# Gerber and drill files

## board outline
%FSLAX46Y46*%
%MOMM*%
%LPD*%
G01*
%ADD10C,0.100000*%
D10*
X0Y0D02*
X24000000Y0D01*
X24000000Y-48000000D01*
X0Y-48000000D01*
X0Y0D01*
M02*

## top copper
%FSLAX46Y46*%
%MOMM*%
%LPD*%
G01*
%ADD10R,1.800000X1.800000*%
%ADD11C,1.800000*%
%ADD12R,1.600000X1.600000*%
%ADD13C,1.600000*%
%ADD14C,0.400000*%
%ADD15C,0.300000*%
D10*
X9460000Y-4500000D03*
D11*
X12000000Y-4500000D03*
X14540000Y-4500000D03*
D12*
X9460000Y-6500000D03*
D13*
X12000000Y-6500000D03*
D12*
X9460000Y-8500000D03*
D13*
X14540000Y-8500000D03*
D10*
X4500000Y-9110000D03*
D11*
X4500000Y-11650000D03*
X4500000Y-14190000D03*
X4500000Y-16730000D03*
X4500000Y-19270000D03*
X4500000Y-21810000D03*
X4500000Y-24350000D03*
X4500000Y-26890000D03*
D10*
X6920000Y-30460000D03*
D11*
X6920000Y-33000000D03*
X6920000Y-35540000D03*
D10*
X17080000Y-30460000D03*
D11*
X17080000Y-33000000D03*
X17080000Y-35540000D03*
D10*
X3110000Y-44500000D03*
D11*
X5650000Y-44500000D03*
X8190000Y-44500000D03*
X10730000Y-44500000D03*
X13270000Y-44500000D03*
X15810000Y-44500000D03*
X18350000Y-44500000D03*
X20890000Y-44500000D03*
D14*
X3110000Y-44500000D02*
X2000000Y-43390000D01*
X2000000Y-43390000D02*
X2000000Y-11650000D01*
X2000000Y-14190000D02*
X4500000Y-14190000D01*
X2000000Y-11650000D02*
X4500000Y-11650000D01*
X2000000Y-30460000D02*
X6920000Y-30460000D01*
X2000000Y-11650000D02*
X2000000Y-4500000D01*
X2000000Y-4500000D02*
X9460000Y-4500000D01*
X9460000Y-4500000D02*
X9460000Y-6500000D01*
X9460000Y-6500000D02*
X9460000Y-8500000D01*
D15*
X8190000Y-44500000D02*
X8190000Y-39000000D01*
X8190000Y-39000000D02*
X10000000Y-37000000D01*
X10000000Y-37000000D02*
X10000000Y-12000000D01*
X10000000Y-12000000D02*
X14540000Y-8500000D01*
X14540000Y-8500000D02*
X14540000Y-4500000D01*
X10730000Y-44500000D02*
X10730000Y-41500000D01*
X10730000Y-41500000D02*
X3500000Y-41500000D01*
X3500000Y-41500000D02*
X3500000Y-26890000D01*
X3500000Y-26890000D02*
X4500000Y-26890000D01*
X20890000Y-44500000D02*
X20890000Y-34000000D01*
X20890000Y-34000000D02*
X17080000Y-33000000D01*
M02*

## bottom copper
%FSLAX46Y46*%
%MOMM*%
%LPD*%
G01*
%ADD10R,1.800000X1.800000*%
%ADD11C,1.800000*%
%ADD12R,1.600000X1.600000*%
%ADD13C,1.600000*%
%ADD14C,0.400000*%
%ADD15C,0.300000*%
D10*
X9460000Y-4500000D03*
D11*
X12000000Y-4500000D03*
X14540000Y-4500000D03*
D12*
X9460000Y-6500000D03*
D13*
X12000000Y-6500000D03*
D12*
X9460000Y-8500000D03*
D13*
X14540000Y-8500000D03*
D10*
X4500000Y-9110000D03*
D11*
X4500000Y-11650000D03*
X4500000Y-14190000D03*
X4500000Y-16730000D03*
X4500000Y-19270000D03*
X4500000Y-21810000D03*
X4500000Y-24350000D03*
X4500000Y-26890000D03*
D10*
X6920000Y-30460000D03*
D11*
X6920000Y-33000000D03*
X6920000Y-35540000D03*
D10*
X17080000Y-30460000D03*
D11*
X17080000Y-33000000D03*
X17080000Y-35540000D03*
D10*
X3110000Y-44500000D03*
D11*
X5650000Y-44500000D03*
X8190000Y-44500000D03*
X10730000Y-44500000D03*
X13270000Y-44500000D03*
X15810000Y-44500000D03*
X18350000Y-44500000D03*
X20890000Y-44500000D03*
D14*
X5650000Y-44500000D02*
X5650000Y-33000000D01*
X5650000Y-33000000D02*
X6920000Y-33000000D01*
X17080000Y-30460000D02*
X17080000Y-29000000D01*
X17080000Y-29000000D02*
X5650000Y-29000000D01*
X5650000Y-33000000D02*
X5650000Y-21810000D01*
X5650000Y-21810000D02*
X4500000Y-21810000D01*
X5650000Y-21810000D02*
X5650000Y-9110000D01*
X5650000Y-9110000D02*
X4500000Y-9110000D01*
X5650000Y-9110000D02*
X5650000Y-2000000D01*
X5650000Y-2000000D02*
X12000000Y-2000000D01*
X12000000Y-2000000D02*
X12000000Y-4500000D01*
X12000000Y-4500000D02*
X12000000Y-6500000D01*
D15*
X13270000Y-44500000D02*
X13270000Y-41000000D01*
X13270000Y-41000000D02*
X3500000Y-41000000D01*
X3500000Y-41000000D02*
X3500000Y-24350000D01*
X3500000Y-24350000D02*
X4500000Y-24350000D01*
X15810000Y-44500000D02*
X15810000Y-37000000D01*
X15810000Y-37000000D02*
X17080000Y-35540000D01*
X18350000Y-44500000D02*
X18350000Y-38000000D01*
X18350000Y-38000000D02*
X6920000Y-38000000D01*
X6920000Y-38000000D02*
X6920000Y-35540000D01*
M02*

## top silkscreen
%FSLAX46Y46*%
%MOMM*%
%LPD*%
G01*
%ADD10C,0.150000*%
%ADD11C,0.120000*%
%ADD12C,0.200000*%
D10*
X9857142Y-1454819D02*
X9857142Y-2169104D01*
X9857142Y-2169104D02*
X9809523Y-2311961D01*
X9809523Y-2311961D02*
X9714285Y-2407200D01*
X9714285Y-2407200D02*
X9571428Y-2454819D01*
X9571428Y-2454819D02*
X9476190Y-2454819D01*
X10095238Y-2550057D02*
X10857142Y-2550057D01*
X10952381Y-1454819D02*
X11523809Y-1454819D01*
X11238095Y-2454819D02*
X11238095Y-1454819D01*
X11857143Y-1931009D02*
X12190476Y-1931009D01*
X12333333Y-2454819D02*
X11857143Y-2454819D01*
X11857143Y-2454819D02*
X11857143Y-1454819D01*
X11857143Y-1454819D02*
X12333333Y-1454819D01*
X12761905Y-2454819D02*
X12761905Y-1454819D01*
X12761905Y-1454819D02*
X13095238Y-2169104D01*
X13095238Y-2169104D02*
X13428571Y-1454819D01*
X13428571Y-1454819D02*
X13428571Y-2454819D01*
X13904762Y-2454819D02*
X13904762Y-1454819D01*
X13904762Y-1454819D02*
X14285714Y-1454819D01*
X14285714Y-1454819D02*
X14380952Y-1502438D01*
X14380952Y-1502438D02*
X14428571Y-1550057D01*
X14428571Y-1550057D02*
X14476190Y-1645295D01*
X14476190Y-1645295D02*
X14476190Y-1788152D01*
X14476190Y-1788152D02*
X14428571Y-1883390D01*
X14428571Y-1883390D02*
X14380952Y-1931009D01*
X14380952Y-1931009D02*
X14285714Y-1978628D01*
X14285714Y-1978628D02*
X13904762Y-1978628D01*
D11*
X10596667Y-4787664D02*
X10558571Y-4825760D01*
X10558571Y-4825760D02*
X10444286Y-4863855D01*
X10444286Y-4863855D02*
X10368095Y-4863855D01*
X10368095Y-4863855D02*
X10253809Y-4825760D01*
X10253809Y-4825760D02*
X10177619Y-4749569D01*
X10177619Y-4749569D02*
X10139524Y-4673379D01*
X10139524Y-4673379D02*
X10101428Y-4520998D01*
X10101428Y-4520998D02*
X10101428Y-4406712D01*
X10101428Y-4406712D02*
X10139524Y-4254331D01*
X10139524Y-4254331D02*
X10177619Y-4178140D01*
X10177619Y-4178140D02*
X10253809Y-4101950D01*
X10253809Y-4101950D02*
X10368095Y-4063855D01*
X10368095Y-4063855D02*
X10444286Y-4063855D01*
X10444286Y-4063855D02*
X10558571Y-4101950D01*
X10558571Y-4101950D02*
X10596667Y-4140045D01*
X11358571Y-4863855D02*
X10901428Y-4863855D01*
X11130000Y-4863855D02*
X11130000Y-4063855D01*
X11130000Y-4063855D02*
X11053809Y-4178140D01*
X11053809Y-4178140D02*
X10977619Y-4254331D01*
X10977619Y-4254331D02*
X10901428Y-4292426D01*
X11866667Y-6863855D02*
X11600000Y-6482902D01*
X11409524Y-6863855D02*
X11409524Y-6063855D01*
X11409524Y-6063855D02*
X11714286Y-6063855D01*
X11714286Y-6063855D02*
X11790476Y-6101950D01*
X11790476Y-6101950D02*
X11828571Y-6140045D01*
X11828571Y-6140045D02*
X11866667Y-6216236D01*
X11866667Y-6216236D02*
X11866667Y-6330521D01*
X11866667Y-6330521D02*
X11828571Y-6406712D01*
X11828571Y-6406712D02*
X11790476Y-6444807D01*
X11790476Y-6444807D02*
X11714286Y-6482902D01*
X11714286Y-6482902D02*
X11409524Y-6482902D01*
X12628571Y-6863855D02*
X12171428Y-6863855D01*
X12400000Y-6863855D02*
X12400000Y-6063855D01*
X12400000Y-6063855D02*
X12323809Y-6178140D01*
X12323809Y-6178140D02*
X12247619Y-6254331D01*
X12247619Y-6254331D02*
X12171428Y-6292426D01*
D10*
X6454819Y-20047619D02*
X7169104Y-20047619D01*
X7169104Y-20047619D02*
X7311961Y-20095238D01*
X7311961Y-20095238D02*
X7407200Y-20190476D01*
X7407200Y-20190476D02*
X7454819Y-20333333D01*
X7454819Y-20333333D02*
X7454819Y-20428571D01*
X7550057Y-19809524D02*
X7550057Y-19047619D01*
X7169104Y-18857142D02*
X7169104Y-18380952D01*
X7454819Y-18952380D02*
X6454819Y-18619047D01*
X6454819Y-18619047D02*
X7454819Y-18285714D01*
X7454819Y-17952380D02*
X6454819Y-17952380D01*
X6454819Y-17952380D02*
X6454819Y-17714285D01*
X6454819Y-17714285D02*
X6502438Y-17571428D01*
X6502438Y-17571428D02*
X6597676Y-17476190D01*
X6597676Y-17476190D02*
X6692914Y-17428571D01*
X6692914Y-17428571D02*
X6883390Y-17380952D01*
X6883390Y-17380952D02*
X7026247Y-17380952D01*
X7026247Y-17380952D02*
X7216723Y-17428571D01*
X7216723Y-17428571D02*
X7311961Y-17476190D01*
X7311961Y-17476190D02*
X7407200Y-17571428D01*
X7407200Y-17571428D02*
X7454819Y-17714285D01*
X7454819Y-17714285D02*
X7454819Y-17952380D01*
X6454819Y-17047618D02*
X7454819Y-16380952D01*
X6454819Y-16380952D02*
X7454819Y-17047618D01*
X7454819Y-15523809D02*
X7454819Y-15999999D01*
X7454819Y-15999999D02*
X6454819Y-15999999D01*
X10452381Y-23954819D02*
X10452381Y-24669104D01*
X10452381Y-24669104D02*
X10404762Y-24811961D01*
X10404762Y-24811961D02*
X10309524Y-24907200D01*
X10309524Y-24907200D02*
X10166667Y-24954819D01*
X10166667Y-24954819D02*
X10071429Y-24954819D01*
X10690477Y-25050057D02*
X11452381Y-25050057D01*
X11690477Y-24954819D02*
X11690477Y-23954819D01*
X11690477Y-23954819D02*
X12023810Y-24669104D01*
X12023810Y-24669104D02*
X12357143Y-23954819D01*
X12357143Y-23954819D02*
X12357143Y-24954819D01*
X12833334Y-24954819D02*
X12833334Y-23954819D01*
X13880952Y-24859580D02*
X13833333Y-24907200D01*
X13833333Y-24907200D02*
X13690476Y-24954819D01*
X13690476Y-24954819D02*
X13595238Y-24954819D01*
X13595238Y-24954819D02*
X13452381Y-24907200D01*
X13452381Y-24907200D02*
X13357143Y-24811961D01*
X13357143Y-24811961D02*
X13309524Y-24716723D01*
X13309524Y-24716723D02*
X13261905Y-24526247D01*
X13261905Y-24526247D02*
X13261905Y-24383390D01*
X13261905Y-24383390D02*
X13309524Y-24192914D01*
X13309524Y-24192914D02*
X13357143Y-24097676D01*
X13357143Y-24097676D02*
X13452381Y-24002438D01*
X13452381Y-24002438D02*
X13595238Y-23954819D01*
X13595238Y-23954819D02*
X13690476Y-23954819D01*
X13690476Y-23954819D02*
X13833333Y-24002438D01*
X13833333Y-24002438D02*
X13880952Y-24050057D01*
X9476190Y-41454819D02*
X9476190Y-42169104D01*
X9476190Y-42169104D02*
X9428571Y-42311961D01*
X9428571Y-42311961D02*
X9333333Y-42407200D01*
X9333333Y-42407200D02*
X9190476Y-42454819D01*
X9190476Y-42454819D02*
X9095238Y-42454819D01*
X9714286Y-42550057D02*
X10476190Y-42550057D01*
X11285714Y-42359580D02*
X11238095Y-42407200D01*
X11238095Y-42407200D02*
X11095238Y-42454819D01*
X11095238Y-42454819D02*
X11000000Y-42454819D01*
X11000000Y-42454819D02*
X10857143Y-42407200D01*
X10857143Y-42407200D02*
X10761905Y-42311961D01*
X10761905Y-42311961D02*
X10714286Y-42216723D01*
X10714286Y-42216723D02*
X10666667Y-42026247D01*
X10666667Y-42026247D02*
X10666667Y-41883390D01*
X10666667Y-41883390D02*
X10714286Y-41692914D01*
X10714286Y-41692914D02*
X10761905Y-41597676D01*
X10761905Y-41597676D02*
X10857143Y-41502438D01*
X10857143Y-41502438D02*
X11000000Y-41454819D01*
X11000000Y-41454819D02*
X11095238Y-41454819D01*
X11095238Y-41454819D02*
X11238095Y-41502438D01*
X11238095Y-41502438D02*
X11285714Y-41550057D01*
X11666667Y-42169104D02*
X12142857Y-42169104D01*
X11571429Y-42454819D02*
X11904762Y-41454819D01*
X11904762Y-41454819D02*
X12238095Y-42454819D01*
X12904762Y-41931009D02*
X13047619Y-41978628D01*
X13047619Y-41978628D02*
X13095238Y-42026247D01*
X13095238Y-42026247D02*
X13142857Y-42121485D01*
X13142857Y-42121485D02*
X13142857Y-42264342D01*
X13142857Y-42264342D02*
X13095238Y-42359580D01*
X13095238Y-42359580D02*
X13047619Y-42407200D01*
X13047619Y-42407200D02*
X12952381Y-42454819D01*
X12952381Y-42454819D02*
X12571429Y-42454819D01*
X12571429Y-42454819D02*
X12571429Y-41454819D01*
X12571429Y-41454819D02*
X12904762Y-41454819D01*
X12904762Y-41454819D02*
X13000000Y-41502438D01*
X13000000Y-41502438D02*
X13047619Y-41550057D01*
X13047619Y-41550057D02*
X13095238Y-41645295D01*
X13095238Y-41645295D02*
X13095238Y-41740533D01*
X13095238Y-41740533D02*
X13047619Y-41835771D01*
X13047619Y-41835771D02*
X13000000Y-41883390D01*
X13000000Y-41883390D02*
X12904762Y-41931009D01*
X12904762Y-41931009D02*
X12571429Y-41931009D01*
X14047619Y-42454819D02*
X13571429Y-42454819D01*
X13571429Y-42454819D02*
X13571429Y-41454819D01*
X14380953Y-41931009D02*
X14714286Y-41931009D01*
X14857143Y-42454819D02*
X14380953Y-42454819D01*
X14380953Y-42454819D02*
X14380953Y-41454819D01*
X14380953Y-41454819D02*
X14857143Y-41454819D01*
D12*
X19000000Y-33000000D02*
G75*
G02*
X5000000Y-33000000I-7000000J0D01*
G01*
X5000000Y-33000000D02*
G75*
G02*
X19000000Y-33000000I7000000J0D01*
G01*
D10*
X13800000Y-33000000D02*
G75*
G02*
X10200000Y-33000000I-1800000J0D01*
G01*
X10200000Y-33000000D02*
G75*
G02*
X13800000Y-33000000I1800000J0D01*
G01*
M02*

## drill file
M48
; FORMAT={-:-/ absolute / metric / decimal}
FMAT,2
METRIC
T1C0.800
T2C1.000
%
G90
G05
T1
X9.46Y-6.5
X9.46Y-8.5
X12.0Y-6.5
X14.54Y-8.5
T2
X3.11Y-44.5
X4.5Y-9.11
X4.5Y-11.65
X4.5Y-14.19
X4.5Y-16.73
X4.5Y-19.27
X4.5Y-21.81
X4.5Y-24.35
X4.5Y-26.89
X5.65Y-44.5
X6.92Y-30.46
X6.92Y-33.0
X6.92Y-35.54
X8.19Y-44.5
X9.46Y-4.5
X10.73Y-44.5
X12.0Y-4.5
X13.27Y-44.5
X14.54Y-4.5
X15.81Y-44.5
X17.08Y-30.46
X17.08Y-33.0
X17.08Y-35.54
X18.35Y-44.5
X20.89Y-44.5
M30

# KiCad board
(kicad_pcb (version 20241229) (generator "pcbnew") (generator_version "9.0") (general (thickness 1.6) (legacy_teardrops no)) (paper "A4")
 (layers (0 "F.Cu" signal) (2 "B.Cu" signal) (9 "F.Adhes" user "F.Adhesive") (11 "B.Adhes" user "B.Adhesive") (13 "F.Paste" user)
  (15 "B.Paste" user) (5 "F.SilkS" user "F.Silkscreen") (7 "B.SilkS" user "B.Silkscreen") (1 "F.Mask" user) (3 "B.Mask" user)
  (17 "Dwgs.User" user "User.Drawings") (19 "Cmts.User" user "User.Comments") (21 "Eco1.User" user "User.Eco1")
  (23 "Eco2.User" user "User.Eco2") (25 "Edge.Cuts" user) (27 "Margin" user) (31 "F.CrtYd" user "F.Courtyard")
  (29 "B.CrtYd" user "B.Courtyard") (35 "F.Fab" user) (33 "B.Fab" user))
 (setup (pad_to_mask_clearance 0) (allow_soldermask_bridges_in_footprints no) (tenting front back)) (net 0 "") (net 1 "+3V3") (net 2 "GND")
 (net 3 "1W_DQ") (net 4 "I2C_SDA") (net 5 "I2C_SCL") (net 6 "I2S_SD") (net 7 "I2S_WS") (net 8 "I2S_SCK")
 (gr_rect (start 0 0) (end 24 48) (stroke (width 0.1) (type solid)) (fill none) (layer "Edge.Cuts"))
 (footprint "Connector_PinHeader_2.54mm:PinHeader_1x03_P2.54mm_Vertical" (layer "F.Cu") (at 12.0 4.5)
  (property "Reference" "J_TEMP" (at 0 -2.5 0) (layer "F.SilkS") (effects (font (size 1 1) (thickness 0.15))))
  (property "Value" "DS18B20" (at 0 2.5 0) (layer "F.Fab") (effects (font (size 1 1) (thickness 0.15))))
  (pad "1" thru_hole rect (at -2.54 0) (size 1.8 1.8) (drill 1.0) (layers "*.Cu" "*.Mask") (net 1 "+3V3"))
  (pad "2" thru_hole circle (at 0 0) (size 1.8 1.8) (drill 1.0) (layers "*.Cu" "*.Mask") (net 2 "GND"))
  (pad "3" thru_hole circle (at 2.54 0) (size 1.8 1.8) (drill 1.0) (layers "*.Cu" "*.Mask") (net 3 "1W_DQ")))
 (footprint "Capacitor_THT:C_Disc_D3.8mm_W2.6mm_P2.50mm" (layer "F.Cu") (at 10.73 6.5)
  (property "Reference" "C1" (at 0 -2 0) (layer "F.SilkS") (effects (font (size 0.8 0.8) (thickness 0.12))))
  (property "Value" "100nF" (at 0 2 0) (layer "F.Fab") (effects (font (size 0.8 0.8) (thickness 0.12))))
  (pad "1" thru_hole rect (at -1.27 0) (size 1.6 1.6) (drill 0.8) (layers "*.Cu" "*.Mask") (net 1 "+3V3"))
  (pad "2" thru_hole circle (at 1.27 0) (size 1.6 1.6) (drill 0.8) (layers "*.Cu" "*.Mask") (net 2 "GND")))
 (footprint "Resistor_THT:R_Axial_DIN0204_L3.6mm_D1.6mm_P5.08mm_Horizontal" (layer "F.Cu") (at 12.0 8.5)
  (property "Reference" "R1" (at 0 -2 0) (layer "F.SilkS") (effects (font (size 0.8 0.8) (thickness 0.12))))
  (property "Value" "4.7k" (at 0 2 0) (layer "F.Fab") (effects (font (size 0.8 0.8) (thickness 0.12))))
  (pad "1" thru_hole rect (at -2.54 0) (size 1.6 1.6) (drill 0.8) (layers "*.Cu" "*.Mask") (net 1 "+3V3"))
  (pad "2" thru_hole circle (at 2.54 0) (size 1.6 1.6) (drill 0.8) (layers "*.Cu" "*.Mask") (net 3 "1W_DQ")))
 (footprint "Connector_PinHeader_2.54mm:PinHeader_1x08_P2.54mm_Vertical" (layer "F.Cu") (at 4.5 18.0)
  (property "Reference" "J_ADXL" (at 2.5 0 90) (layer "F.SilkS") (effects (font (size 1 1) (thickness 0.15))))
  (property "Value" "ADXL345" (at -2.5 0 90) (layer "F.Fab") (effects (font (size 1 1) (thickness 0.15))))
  (pad "1" thru_hole rect (at 0 -8.89) (size 1.8 1.8) (drill 1.0) (layers "*.Cu" "*.Mask") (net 2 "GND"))
  (pad "2" thru_hole circle (at 0 -6.35) (size 1.8 1.8) (drill 1.0) (layers "*.Cu" "*.Mask") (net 1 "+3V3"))
  (pad "3" thru_hole circle (at 0 -3.81) (size 1.8 1.8) (drill 1.0) (layers "*.Cu" "*.Mask") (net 1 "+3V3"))
  (pad "4" thru_hole circle (at 0 -1.27) (size 1.8 1.8) (drill 1.0) (layers "*.Cu" "*.Mask") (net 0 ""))
  (pad "5" thru_hole circle (at 0 1.27) (size 1.8 1.8) (drill 1.0) (layers "*.Cu" "*.Mask") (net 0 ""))
  (pad "6" thru_hole circle (at 0 3.81) (size 1.8 1.8) (drill 1.0) (layers "*.Cu" "*.Mask") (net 2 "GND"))
  (pad "7" thru_hole circle (at 0 6.35) (size 1.8 1.8) (drill 1.0) (layers "*.Cu" "*.Mask") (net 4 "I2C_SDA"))
  (pad "8" thru_hole circle (at 0 8.89) (size 1.8 1.8) (drill 1.0) (layers "*.Cu" "*.Mask") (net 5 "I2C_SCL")))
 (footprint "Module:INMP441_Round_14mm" (layer "F.Cu") (at 12.0 33.0)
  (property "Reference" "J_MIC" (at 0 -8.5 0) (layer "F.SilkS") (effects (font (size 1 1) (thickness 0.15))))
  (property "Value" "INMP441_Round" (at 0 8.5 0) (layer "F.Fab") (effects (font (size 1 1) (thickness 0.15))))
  (fp_circle (center 0 0) (end 7.0 0) (stroke (width 0.2) (type solid)) (layer "F.SilkS"))
  (fp_circle (center 0 0) (end 1.8 0) (stroke (width 0.15) (type solid)) (layer "F.SilkS"))
  (pad "1" thru_hole rect (at -5.08 -2.54) (size 1.8 1.8) (drill 1.0) (layers "*.Cu" "*.Mask") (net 1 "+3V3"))
  (pad "2" thru_hole circle (at -5.08 0) (size 1.8 1.8) (drill 1.0) (layers "*.Cu" "*.Mask") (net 2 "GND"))
  (pad "3" thru_hole circle (at -5.08 2.54) (size 1.8 1.8) (drill 1.0) (layers "*.Cu" "*.Mask") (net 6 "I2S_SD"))
  (pad "4" thru_hole rect (at 5.08 -2.54) (size 1.8 1.8) (drill 1.0) (layers "*.Cu" "*.Mask") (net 2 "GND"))
  (pad "5" thru_hole circle (at 5.08 0) (size 1.8 1.8) (drill 1.0) (layers "*.Cu" "*.Mask") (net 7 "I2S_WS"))
  (pad "6" thru_hole circle (at 5.08 2.54) (size 1.8 1.8) (drill 1.0) (layers "*.Cu" "*.Mask") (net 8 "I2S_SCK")))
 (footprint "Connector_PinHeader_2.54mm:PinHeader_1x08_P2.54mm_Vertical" (layer "F.Cu") (at 12.0 44.5)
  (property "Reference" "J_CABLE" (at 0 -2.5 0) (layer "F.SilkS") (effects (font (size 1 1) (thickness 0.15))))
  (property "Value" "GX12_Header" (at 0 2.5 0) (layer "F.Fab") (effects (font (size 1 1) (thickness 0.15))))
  (pad "1" thru_hole rect (at -8.89 0) (size 1.8 1.8) (drill 1.0) (layers "*.Cu" "*.Mask") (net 1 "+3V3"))
  (pad "2" thru_hole circle (at -6.35 0) (size 1.8 1.8) (drill 1.0) (layers "*.Cu" "*.Mask") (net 2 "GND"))
  (pad "3" thru_hole circle (at -3.81 0) (size 1.8 1.8) (drill 1.0) (layers "*.Cu" "*.Mask") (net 3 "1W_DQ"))
  (pad "4" thru_hole circle (at -1.27 0) (size 1.8 1.8) (drill 1.0) (layers "*.Cu" "*.Mask") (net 5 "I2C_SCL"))
  (pad "5" thru_hole circle (at 1.27 0) (size 1.8 1.8) (drill 1.0) (layers "*.Cu" "*.Mask") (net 4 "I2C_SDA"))
  (pad "6" thru_hole circle (at 3.81 0) (size 1.8 1.8) (drill 1.0) (layers "*.Cu" "*.Mask") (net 8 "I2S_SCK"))
  (pad "7" thru_hole circle (at 6.35 0) (size 1.8 1.8) (drill 1.0) (layers "*.Cu" "*.Mask") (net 6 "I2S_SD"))
  (pad "8" thru_hole circle (at 8.89 0) (size 1.8 1.8) (drill 1.0) (layers "*.Cu" "*.Mask") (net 7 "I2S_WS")))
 (segment (start 3.11 44.5) (end 2.0 43.39) (width 0.4) (layer "F.Cu") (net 1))
 (segment (start 2.0 43.39) (end 2.0 11.65) (width 0.4) (layer "F.Cu") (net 1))
 (segment (start 2.0 14.19) (end 4.5 14.19) (width 0.4) (layer "F.Cu") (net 1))
 (segment (start 2.0 11.65) (end 4.5 11.65) (width 0.4) (layer "F.Cu") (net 1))
 (segment (start 2.0 30.46) (end 6.92 30.46) (width 0.4) (layer "F.Cu") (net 1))
 (segment (start 2.0 11.65) (end 2.0 4.5) (width 0.4) (layer "F.Cu") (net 1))
 (segment (start 2.0 4.5) (end 9.46 4.5) (width 0.4) (layer "F.Cu") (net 1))
 (segment (start 9.46 4.5) (end 9.46 6.5) (width 0.4) (layer "F.Cu") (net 1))
 (segment (start 9.46 6.5) (end 9.46 8.5) (width 0.4) (layer "F.Cu") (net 1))
 (segment (start 5.65 44.5) (end 5.65 33.0) (width 0.4) (layer "B.Cu") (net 2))
 (segment (start 5.65 33.0) (end 6.92 33.0) (width 0.4) (layer "B.Cu") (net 2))
 (segment (start 17.08 30.46) (end 17.08 29.0) (width 0.4) (layer "B.Cu") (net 2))
 (segment (start 17.08 29.0) (end 5.65 29.0) (width 0.4) (layer "B.Cu") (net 2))
 (segment (start 5.65 33.0) (end 5.65 21.81) (width 0.4) (layer "B.Cu") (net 2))
 (segment (start 5.65 21.81) (end 4.5 21.81) (width 0.4) (layer "B.Cu") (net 2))
 (segment (start 5.65 21.81) (end 5.65 9.11) (width 0.4) (layer "B.Cu") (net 2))
 (segment (start 5.65 9.11) (end 4.5 9.11) (width 0.4) (layer "B.Cu") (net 2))
 (segment (start 5.65 9.11) (end 5.65 2.0) (width 0.4) (layer "B.Cu") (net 2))
 (segment (start 5.65 2.0) (end 12.0 2.0) (width 0.4) (layer "B.Cu") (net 2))
 (segment (start 12.0 2.0) (end 12.0 4.5) (width 0.4) (layer "B.Cu") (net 2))
 (segment (start 12.0 4.5) (end 12.0 6.5) (width 0.4) (layer "B.Cu") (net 2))
 (segment (start 8.19 44.5) (end 8.19 39.0) (width 0.3) (layer "F.Cu") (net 3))
 (segment (start 8.19 39.0) (end 10.0 37.0) (width 0.3) (layer "F.Cu") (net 3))
 (segment (start 10.0 37.0) (end 10.0 12.0) (width 0.3) (layer "F.Cu") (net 3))
 (segment (start 10.0 12.0) (end 14.54 8.5) (width 0.3) (layer "F.Cu") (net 3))
 (segment (start 14.54 8.5) (end 14.54 4.5) (width 0.3) (layer "F.Cu") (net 3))
 (segment (start 10.73 44.5) (end 10.73 41.5) (width 0.3) (layer "F.Cu") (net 5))
 (segment (start 10.73 41.5) (end 3.5 41.5) (width 0.3) (layer "F.Cu") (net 5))
 (segment (start 3.5 41.5) (end 3.5 26.89) (width 0.3) (layer "F.Cu") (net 5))
 (segment (start 3.5 26.89) (end 4.5 26.89) (width 0.3) (layer "F.Cu") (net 5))
 (segment (start 13.27 44.5) (end 13.27 41.0) (width 0.3) (layer "B.Cu") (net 4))
 (segment (start 13.27 41.0) (end 3.5 41.0) (width 0.3) (layer "B.Cu") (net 4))
 (segment (start 3.5 41.0) (end 3.5 24.35) (width 0.3) (layer "B.Cu") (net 4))
 (segment (start 3.5 24.35) (end 4.5 24.35) (width 0.3) (layer "B.Cu") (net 4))
 (segment (start 15.81 44.5) (end 15.81 37.0) (width 0.3) (layer "B.Cu") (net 8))
 (segment (start 15.81 37.0) (end 17.08 35.54) (width 0.3) (layer "B.Cu") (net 8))
 (segment (start 18.35 44.5) (end 18.35 38.0) (width 0.3) (layer "B.Cu") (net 6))
 (segment (start 18.35 38.0) (end 6.92 38.0) (width 0.3) (layer "B.Cu") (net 6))
 (segment (start 6.92 38.0) (end 6.92 35.54) (width 0.3) (layer "B.Cu") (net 6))
 (segment (start 20.89 44.5) (end 20.89 34.0) (width 0.3) (layer "F.Cu") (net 7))
 (segment (start 20.89 34.0) (end 17.08 33.0) (width 0.3) (layer "F.Cu") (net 7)))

